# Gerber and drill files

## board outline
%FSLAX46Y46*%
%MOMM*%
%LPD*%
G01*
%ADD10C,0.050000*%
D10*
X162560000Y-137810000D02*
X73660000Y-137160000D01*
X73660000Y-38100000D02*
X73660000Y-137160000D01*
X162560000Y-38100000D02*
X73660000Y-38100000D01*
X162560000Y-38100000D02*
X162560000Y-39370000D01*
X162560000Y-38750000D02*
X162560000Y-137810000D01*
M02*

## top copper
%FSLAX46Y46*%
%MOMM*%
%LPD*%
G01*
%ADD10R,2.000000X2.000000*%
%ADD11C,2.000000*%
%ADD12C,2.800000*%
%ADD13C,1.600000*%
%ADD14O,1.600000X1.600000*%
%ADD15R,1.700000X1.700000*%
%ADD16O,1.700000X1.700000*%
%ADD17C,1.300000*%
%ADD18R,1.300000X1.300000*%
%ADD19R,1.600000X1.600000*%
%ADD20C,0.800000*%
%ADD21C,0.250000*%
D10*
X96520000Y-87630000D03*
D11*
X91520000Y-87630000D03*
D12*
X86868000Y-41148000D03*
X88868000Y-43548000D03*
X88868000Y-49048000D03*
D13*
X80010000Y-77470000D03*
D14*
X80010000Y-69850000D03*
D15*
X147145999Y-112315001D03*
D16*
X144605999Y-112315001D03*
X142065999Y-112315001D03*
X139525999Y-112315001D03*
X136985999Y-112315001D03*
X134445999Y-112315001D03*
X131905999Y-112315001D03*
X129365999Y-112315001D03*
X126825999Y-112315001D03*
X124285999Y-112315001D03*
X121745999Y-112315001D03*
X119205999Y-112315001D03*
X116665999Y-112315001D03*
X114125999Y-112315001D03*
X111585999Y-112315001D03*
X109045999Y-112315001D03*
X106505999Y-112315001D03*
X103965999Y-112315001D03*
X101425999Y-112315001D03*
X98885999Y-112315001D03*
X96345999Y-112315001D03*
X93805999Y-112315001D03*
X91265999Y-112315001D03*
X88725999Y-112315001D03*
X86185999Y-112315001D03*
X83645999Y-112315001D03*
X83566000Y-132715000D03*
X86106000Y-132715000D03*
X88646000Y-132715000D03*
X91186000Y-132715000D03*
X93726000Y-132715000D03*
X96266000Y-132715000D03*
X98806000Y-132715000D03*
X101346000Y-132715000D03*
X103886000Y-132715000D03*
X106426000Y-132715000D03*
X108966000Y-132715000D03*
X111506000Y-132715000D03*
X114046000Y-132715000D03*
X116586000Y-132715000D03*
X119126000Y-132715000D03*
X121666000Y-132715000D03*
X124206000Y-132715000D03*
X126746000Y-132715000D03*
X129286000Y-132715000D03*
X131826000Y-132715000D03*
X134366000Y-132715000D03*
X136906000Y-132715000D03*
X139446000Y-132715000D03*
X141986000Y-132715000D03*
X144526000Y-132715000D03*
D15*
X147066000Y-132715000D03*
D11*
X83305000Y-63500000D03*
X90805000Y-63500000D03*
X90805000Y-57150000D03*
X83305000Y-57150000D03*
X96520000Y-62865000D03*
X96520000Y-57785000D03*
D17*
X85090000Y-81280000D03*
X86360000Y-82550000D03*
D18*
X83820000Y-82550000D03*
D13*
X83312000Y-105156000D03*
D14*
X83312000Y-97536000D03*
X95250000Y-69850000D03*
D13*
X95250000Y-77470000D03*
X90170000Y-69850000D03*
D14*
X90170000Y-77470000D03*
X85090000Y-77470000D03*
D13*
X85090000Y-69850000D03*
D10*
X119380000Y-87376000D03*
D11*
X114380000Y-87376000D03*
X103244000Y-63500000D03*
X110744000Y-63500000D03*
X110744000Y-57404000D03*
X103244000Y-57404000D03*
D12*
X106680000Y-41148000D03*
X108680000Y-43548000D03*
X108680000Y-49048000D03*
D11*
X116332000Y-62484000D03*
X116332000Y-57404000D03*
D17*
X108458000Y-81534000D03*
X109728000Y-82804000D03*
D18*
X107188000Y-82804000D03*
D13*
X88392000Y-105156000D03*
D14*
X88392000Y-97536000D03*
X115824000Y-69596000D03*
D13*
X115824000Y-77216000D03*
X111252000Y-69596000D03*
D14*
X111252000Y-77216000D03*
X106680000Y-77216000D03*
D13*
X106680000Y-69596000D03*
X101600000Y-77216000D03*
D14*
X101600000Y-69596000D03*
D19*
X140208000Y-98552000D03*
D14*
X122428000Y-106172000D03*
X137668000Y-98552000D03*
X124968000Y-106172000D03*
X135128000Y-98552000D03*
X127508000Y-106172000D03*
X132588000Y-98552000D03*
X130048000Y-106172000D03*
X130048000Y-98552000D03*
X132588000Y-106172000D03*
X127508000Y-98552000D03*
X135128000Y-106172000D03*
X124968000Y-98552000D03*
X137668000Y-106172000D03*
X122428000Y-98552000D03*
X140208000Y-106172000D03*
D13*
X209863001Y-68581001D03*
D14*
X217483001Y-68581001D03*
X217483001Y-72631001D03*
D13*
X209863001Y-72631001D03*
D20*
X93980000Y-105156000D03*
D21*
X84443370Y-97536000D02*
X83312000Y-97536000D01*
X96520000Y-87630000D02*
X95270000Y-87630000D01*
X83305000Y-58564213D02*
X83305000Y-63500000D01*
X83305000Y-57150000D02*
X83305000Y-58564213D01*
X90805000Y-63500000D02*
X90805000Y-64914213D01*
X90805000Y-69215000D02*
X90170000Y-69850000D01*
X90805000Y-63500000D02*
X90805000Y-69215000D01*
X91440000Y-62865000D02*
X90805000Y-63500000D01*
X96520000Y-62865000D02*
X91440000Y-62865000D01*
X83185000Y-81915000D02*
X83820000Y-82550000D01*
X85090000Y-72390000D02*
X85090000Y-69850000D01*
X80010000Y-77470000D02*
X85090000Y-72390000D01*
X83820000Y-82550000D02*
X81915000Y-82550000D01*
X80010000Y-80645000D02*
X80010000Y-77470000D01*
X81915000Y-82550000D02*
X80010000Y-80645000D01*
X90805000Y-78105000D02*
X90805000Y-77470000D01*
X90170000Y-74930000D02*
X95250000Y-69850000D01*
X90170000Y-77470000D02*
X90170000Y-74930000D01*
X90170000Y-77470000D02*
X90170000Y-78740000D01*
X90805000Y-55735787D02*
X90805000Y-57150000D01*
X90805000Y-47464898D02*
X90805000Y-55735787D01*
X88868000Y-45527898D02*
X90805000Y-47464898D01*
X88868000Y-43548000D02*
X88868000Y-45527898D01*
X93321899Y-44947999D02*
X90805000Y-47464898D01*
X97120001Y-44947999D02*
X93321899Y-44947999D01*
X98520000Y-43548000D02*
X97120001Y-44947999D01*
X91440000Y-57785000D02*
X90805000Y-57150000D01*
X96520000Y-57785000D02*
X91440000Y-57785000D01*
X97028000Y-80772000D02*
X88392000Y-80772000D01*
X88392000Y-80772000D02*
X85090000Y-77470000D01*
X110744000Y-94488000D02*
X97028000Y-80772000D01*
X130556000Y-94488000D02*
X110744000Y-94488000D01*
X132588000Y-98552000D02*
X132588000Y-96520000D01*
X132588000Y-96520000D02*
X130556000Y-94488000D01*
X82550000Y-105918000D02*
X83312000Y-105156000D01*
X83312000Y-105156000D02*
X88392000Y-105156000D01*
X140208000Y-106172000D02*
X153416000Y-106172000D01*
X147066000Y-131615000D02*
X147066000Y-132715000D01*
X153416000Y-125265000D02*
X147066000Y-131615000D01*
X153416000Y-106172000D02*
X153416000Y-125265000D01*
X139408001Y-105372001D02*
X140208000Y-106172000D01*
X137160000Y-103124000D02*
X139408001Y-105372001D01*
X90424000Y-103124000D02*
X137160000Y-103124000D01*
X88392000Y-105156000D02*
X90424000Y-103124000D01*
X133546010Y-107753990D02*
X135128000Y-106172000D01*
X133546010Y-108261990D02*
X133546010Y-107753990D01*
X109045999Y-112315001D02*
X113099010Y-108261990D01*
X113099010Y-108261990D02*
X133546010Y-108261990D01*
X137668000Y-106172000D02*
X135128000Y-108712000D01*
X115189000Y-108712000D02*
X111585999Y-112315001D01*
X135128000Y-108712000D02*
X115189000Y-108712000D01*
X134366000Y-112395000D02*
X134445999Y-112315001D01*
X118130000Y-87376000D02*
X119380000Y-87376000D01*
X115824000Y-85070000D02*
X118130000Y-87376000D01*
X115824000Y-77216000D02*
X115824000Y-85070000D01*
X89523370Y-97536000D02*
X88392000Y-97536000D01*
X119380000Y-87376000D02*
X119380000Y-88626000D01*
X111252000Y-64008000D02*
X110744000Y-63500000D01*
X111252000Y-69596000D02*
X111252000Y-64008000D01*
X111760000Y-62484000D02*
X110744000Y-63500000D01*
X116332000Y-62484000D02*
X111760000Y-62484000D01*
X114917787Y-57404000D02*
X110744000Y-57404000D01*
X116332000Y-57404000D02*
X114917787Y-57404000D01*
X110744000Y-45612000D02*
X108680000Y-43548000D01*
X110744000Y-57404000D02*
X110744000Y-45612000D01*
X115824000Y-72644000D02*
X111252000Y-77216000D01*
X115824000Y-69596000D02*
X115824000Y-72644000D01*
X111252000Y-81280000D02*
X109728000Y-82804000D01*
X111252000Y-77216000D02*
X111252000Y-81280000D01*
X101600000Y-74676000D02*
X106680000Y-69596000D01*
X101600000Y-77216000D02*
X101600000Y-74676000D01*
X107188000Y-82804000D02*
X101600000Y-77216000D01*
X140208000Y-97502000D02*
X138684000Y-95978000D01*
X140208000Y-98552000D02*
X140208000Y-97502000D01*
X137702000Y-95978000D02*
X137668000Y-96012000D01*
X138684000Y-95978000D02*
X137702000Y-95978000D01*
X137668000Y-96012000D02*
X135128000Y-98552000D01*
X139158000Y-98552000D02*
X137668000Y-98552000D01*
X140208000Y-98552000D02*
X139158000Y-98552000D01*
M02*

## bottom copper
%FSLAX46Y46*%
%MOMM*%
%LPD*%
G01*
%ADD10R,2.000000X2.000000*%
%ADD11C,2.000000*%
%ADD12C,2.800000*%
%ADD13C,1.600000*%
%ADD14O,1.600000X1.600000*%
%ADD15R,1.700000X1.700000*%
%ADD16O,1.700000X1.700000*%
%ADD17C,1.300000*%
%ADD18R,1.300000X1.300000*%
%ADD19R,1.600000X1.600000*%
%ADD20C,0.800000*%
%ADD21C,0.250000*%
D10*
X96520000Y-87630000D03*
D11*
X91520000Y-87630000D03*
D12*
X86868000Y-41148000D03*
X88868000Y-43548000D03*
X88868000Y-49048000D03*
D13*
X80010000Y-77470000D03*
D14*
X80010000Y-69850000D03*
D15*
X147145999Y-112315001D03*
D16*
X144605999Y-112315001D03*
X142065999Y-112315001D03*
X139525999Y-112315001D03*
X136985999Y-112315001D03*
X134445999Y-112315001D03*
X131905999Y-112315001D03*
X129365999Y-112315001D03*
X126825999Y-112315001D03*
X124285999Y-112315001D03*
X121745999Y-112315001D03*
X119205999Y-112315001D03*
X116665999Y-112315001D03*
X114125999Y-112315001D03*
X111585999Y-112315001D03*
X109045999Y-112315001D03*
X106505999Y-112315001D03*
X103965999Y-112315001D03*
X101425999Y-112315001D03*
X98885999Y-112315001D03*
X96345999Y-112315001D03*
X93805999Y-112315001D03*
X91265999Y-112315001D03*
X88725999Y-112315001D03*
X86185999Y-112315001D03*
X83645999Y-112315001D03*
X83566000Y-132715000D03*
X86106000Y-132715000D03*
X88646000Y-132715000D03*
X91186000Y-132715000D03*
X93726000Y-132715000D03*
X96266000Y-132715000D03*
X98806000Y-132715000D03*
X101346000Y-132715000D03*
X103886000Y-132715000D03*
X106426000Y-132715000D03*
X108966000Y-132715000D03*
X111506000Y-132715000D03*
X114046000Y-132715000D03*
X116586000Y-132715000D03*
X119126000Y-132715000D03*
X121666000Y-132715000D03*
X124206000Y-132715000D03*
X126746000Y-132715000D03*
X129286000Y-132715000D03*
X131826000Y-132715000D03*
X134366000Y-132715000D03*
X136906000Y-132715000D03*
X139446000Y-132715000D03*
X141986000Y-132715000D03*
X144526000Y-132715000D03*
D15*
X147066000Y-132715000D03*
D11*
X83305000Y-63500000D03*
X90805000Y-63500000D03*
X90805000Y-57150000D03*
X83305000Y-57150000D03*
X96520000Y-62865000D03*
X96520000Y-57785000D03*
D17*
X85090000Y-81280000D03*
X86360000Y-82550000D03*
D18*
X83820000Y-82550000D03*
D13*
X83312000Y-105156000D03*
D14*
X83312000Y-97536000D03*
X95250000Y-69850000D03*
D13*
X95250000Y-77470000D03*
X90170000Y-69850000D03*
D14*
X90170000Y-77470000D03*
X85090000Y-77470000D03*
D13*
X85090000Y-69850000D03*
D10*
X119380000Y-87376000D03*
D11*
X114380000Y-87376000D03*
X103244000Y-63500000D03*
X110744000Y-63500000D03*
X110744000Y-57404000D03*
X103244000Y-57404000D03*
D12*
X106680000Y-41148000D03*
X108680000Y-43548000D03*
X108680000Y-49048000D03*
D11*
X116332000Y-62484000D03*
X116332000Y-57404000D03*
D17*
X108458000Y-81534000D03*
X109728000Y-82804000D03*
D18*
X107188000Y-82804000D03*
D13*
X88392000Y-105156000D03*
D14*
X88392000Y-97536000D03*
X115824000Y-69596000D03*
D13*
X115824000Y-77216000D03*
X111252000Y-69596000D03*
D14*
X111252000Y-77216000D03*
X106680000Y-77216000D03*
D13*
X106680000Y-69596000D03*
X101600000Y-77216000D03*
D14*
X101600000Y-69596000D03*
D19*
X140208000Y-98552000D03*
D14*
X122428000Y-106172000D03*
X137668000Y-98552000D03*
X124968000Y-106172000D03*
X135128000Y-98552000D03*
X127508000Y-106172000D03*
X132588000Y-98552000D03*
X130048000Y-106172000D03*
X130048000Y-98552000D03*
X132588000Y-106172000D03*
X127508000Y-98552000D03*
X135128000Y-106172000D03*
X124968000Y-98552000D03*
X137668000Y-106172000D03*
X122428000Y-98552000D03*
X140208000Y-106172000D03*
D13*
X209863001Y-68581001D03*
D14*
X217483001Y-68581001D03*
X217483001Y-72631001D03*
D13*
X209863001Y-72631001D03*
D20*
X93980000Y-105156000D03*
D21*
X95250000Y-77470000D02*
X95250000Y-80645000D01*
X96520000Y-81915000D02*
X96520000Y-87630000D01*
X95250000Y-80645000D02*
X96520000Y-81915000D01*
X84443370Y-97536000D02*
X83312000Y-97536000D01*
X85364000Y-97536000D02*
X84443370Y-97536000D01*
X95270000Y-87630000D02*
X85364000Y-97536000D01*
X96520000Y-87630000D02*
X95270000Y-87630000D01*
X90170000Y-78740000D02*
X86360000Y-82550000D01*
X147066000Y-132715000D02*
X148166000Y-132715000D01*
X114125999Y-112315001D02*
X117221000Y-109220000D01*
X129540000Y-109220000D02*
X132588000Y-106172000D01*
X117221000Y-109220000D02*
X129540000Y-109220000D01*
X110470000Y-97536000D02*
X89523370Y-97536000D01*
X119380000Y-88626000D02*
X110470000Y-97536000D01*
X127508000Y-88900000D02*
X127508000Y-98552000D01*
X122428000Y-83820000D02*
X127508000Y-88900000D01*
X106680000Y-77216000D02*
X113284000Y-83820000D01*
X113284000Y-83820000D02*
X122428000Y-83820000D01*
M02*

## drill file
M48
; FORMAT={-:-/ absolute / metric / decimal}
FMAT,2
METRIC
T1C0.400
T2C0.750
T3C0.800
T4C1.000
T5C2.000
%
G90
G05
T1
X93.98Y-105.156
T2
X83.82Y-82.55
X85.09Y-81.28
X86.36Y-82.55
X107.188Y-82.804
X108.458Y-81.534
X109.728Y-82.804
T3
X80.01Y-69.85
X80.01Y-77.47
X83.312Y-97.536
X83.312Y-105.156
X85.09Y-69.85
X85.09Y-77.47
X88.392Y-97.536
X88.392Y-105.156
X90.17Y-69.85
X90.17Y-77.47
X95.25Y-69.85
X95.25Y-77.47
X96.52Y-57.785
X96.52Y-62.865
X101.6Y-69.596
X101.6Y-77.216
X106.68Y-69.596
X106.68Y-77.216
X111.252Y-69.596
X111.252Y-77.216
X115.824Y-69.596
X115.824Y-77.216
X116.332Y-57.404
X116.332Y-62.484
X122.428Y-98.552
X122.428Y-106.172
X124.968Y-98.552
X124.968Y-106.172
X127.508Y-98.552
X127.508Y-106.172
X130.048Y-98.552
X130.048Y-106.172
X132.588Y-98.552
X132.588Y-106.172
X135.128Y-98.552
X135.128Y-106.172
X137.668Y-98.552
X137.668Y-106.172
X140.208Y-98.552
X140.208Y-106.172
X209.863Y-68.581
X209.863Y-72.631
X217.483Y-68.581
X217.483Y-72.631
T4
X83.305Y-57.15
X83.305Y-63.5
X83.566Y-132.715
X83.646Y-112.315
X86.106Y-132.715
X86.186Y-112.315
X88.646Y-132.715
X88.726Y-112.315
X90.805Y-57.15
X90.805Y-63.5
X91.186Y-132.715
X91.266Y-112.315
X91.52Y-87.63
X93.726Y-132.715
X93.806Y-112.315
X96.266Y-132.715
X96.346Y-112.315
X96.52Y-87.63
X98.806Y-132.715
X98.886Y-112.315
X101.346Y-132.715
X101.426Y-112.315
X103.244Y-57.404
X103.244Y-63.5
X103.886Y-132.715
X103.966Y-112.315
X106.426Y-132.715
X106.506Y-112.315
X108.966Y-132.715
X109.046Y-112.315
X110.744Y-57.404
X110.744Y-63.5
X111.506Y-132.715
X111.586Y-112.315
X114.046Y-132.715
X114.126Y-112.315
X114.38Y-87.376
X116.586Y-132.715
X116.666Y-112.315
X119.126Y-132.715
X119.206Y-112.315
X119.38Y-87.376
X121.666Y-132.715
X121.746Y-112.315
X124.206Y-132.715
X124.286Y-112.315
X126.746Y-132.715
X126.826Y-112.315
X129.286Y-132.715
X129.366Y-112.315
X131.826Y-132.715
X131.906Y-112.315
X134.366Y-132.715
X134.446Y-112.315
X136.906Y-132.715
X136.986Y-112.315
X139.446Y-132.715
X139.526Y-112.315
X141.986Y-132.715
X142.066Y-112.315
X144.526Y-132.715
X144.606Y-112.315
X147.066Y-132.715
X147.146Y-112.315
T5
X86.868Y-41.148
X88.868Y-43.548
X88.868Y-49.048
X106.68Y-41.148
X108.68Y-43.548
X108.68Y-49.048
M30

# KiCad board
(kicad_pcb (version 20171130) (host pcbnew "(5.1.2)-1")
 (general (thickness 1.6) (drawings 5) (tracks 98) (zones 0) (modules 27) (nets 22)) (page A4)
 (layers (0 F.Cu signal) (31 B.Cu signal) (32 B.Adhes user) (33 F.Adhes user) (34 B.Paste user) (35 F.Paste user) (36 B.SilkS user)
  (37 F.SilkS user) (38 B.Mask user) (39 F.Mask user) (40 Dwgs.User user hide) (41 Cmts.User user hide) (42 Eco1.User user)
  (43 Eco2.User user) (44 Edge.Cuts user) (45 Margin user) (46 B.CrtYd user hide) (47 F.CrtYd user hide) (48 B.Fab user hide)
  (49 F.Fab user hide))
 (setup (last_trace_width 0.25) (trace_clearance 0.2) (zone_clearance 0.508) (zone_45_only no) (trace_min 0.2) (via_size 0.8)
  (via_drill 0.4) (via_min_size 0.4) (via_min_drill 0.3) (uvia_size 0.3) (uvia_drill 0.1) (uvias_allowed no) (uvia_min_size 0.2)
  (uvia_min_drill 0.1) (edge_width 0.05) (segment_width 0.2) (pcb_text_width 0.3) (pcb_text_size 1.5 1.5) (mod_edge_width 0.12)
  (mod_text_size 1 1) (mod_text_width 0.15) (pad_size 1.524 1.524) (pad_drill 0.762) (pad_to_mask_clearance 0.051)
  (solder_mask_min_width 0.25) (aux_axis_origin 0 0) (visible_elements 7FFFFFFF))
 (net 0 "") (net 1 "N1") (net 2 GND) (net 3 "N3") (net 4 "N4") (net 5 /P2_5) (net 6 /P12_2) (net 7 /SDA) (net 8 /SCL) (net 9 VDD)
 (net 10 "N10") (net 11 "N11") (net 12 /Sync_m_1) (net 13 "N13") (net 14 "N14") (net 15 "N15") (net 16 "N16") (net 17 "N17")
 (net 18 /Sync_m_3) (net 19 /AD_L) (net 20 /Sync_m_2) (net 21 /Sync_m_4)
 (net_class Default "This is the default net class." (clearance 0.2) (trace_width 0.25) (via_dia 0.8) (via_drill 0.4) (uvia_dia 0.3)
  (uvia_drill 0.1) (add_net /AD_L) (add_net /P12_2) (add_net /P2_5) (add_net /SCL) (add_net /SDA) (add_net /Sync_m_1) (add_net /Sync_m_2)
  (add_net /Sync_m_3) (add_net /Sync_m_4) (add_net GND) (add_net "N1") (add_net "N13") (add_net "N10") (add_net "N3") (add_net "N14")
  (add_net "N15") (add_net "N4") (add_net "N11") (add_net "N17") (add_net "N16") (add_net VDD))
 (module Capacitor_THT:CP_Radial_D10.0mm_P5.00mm (layer F.Cu) (at 96.52 87.63 180)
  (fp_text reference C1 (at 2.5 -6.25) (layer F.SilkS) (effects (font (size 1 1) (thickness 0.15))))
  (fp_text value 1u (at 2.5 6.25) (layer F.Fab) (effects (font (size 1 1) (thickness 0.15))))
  (pad 1 thru_hole rect (at 0 0 180) (size 2 2) (drill 1) (layers *.Cu *.Mask) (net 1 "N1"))
  (pad 2 thru_hole circle (at 5 0 180) (size 2 2) (drill 1) (layers *.Cu *.Mask) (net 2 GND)))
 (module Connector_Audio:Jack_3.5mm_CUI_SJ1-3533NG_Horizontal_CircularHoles (layer F.Cu) (at 86.868 41.148)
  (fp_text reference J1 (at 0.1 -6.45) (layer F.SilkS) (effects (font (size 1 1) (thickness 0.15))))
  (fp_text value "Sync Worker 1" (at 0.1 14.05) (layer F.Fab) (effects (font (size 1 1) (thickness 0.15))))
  (pad S thru_hole circle (at 0 0) (size 2.8 2.8) (drill 2) (layers *.Cu *.Mask) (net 2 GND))
  (pad T thru_hole circle (at 2 2.4) (size 2.8 2.8) (drill 2) (layers *.Cu *.Mask) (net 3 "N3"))
  (pad R thru_hole circle (at 2 7.9) (size 2.8 2.8) (drill 2) (layers *.Cu *.Mask)))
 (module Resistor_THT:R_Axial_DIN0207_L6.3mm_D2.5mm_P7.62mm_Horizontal (layer F.Cu) (at 80.01 77.47 90)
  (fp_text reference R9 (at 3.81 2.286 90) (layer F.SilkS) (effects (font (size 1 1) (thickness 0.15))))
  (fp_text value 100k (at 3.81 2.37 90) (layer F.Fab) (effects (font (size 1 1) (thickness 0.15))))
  (pad 1 thru_hole circle (at 0 0 90) (size 1.6 1.6) (drill 0.8) (layers *.Cu *.Mask) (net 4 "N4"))
  (pad 2 thru_hole oval (at 7.62 0 90) (size 1.6 1.6) (drill 0.8) (layers *.Cu *.Mask) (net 2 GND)))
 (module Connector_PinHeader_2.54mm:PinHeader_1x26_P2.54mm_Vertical (layer F.Cu) (at 147.145999 112.315001 270)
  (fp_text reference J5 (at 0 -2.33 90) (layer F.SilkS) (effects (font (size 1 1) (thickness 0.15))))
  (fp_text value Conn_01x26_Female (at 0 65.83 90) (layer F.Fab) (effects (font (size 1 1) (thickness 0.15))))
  (pad 1 thru_hole rect (at 0 0 270) (size 1.7 1.7) (drill 1) (layers *.Cu *.Mask))
  (pad 2 thru_hole oval (at 0 2.54 270) (size 1.7 1.7) (drill 1) (layers *.Cu *.Mask))
  (pad 3 thru_hole oval (at 0 5.08 270) (size 1.7 1.7) (drill 1) (layers *.Cu *.Mask))
  (pad 4 thru_hole oval (at 0 7.62 270) (size 1.7 1.7) (drill 1) (layers *.Cu *.Mask))
  (pad 5 thru_hole oval (at 0 10.16 270) (size 1.7 1.7) (drill 1) (layers *.Cu *.Mask))
  (pad 6 thru_hole oval (at 0 12.7 270) (size 1.7 1.7) (drill 1) (layers *.Cu *.Mask) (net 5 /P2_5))
  (pad 7 thru_hole oval (at 0 15.24 270) (size 1.7 1.7) (drill 1) (layers *.Cu *.Mask))
  (pad 8 thru_hole oval (at 0 17.78 270) (size 1.7 1.7) (drill 1) (layers *.Cu *.Mask))
  (pad 9 thru_hole oval (at 0 20.32 270) (size 1.7 1.7) (drill 1) (layers *.Cu *.Mask))
  (pad 10 thru_hole oval (at 0 22.86 270) (size 1.7 1.7) (drill 1) (layers *.Cu *.Mask))
  (pad 11 thru_hole oval (at 0 25.4 270) (size 1.7 1.7) (drill 1) (layers *.Cu *.Mask))
  (pad 12 thru_hole oval (at 0 27.94 270) (size 1.7 1.7) (drill 1) (layers *.Cu *.Mask))
  (pad 13 thru_hole oval (at 0 30.48 270) (size 1.7 1.7) (drill 1) (layers *.Cu *.Mask))
  (pad 14 thru_hole oval (at 0 33.02 270) (size 1.7 1.7) (drill 1) (layers *.Cu *.Mask) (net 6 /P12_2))
  (pad 15 thru_hole oval (at 0 35.56 270) (size 1.7 1.7) (drill 1) (layers *.Cu *.Mask) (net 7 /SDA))
  (pad 16 thru_hole oval (at 0 38.1 270) (size 1.7 1.7) (drill 1) (layers *.Cu *.Mask) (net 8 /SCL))
  (pad 17 thru_hole oval (at 0 40.64 270) (size 1.7 1.7) (drill 1) (layers *.Cu *.Mask))
  (pad 18 thru_hole oval (at 0 43.18 270) (size 1.7 1.7) (drill 1) (layers *.Cu *.Mask))
  (pad 19 thru_hole oval (at 0 45.72 270) (size 1.7 1.7) (drill 1) (layers *.Cu *.Mask))
  (pad 20 thru_hole oval (at 0 48.26 270) (size 1.7 1.7) (drill 1) (layers *.Cu *.Mask))
  (pad 21 thru_hole oval (at 0 50.8 270) (size 1.7 1.7) (drill 1) (layers *.Cu *.Mask))
  (pad 22 thru_hole oval (at 0 53.34 270) (size 1.7 1.7) (drill 1) (layers *.Cu *.Mask))
  (pad 23 thru_hole oval (at 0 55.88 270) (size 1.7 1.7) (drill 1) (layers *.Cu *.Mask))
  (pad 24 thru_hole oval (at 0 58.42 270) (size 1.7 1.7) (drill 1) (layers *.Cu *.Mask))
  (pad 25 thru_hole oval (at 0 60.96 270) (size 1.7 1.7) (drill 1) (layers *.Cu *.Mask) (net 2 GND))
  (pad 26 thru_hole oval (at 0 63.5 270) (size 1.7 1.7) (drill 1) (layers *.Cu *.Mask)))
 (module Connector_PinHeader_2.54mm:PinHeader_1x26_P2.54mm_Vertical (layer F.Cu) (at 147.066 132.715 270)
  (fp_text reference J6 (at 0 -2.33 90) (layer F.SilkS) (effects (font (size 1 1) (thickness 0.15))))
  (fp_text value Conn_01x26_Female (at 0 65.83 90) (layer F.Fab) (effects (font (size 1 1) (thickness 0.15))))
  (pad 26 thru_hole oval (at 0 63.5 270) (size 1.7 1.7) (drill 1) (layers *.Cu *.Mask) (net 2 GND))
  (pad 25 thru_hole oval (at 0 60.96 270) (size 1.7 1.7) (drill 1) (layers *.Cu *.Mask))
  (pad 24 thru_hole oval (at 0 58.42 270) (size 1.7 1.7) (drill 1) (layers *.Cu *.Mask))
  (pad 23 thru_hole oval (at 0 55.88 270) (size 1.7 1.7) (drill 1) (layers *.Cu *.Mask))
  (pad 22 thru_hole oval (at 0 53.34 270) (size 1.7 1.7) (drill 1) (layers *.Cu *.Mask))
  (pad 21 thru_hole oval (at 0 50.8 270) (size 1.7 1.7) (drill 1) (layers *.Cu *.Mask))
  (pad 20 thru_hole oval (at 0 48.26 270) (size 1.7 1.7) (drill 1) (layers *.Cu *.Mask))
  (pad 19 thru_hole oval (at 0 45.72 270) (size 1.7 1.7) (drill 1) (layers *.Cu *.Mask))
  (pad 18 thru_hole oval (at 0 43.18 270) (size 1.7 1.7) (drill 1) (layers *.Cu *.Mask))
  (pad 17 thru_hole oval (at 0 40.64 270) (size 1.7 1.7) (drill 1) (layers *.Cu *.Mask))
  (pad 16 thru_hole oval (at 0 38.1 270) (size 1.7 1.7) (drill 1) (layers *.Cu *.Mask))
  (pad 15 thru_hole oval (at 0 35.56 270) (size 1.7 1.7) (drill 1) (layers *.Cu *.Mask))
  (pad 14 thru_hole oval (at 0 33.02 270) (size 1.7 1.7) (drill 1) (layers *.Cu *.Mask))
  (pad 13 thru_hole oval (at 0 30.48 270) (size 1.7 1.7) (drill 1) (layers *.Cu *.Mask))
  (pad 12 thru_hole oval (at 0 27.94 270) (size 1.7 1.7) (drill 1) (layers *.Cu *.Mask))
  (pad 11 thru_hole oval (at 0 25.4 270) (size 1.7 1.7) (drill 1) (layers *.Cu *.Mask))
  (pad 10 thru_hole oval (at 0 22.86 270) (size 1.7 1.7) (drill 1) (layers *.Cu *.Mask))
  (pad 9 thru_hole oval (at 0 20.32 270) (size 1.7 1.7) (drill 1) (layers *.Cu *.Mask))
  (pad 8 thru_hole oval (at 0 17.78 270) (size 1.7 1.7) (drill 1) (layers *.Cu *.Mask))
  (pad 7 thru_hole oval (at 0 15.24 270) (size 1.7 1.7) (drill 1) (layers *.Cu *.Mask))
  (pad 6 thru_hole oval (at 0 12.7 270) (size 1.7 1.7) (drill 1) (layers *.Cu *.Mask) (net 5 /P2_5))
  (pad 5 thru_hole oval (at 0 10.16 270) (size 1.7 1.7) (drill 1) (layers *.Cu *.Mask))
  (pad 4 thru_hole oval (at 0 7.62 270) (size 1.7 1.7) (drill 1) (layers *.Cu *.Mask))
  (pad 3 thru_hole oval (at 0 5.08 270) (size 1.7 1.7) (drill 1) (layers *.Cu *.Mask))
  (pad 2 thru_hole oval (at 0 2.54 270) (size 1.7 1.7) (drill 1) (layers *.Cu *.Mask) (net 2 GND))
  (pad 1 thru_hole rect (at 0 0 270) (size 1.7 1.7) (drill 1) (layers *.Cu *.Mask) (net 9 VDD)))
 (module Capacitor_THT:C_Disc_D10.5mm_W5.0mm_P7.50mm (layer F.Cu) (at 90.805 63.5 180)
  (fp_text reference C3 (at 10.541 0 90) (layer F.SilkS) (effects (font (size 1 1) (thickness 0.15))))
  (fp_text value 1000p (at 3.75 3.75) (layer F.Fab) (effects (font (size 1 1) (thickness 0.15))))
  (pad 2 thru_hole circle (at 7.5 0 180) (size 2 2) (drill 1) (layers *.Cu *.Mask) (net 2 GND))
  (pad 1 thru_hole circle (at 0 0 180) (size 2 2) (drill 1) (layers *.Cu *.Mask) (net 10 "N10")))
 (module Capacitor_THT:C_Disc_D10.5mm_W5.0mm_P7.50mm (layer F.Cu) (at 90.805 57.15 180)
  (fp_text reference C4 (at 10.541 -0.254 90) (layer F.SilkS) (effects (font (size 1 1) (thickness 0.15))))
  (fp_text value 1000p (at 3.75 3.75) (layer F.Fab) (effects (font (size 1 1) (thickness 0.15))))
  (pad 1 thru_hole circle (at 0 0 180) (size 2 2) (drill 1) (layers *.Cu *.Mask) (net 3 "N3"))
  (pad 2 thru_hole circle (at 7.5 0 180) (size 2 2) (drill 1) (layers *.Cu *.Mask) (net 2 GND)))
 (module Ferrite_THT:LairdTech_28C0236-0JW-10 (layer F.Cu) (at 96.52 57.785 270)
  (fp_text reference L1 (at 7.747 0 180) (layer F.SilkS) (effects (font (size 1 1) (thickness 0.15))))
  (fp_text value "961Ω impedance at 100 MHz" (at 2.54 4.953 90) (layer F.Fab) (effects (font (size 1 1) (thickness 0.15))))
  (pad 2 thru_hole circle (at 5.08 0 270) (size 2 2) (drill 0.8) (layers *.Cu *.Mask) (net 10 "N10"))
  (pad 1 thru_hole circle (at 0 0 270) (size 2 2) (drill 0.8) (layers *.Cu *.Mask) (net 3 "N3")))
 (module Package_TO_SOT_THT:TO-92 (layer F.Cu) (at 83.82 82.55)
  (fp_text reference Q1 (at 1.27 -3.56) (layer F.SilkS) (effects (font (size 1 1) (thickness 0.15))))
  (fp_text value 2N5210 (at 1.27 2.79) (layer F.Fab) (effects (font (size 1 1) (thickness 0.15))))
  (pad 2 thru_hole circle (at 1.27 -1.27 90) (size 1.3 1.3) (drill 0.75) (layers *.Cu *.Mask) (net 2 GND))
  (pad 3 thru_hole circle (at 2.54 0 90) (size 1.3 1.3) (drill 0.75) (layers *.Cu *.Mask) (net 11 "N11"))
  (pad 1 thru_hole rect (at 0 0 90) (size 1.3 1.3) (drill 0.75) (layers *.Cu *.Mask) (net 4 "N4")))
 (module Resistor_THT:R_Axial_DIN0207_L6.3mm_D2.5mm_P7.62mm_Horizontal (layer F.Cu) (at 83.312 105.156 90)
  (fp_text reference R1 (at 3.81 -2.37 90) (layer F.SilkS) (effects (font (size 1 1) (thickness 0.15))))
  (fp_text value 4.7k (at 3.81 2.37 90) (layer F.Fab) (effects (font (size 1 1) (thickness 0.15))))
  (pad 1 thru_hole circle (at 0 0 90) (size 1.6 1.6) (drill 0.8) (layers *.Cu *.Mask) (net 9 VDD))
  (pad 2 thru_hole oval (at 7.62 0 90) (size 1.6 1.6) (drill 0.8) (layers *.Cu *.Mask) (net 1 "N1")))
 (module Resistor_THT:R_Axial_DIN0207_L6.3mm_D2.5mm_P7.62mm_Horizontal (layer F.Cu) (at 95.25 77.47 90)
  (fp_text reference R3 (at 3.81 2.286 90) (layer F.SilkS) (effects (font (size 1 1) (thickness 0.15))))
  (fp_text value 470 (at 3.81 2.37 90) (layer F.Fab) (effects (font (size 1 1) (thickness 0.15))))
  (pad 2 thru_hole oval (at 7.62 0 90) (size 1.6 1.6) (drill 0.8) (layers *.Cu *.Mask) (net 11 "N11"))
  (pad 1 thru_hole circle (at 0 0 90) (size 1.6 1.6) (drill 0.8) (layers *.Cu *.Mask) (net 1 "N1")))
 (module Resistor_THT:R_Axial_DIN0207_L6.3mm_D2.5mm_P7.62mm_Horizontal (layer F.Cu) (at 90.17 69.85 270)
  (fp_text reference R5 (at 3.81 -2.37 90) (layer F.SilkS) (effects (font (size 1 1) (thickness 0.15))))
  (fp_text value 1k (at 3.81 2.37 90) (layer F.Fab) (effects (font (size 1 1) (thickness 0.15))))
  (pad 1 thru_hole circle (at 0 0 270) (size 1.6 1.6) (drill 0.8) (layers *.Cu *.Mask) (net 10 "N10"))
  (pad 2 thru_hole oval (at 7.62 0 270) (size 1.6 1.6) (drill 0.8) (layers *.Cu *.Mask) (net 11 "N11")))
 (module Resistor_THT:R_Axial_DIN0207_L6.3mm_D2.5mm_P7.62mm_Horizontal (layer F.Cu) (at 85.09 69.85 270)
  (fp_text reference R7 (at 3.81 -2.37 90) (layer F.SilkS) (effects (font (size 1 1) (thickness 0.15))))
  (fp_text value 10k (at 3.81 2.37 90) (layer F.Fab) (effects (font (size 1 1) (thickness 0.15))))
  (pad 2 thru_hole oval (at 7.62 0 270) (size 1.6 1.6) (drill 0.8) (layers *.Cu *.Mask) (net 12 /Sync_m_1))
  (pad 1 thru_hole circle (at 0 0 270) (size 1.6 1.6) (drill 0.8) (layers *.Cu *.Mask) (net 4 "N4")))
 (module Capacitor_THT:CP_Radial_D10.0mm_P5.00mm (layer F.Cu) (at 119.38 87.376 180)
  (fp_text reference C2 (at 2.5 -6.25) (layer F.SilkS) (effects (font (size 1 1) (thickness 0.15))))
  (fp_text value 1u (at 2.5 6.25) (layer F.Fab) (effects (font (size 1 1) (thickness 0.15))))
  (pad 1 thru_hole rect (at 0 0 180) (size 2 2) (drill 1) (layers *.Cu *.Mask) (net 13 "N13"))
  (pad 2 thru_hole circle (at 5 0 180) (size 2 2) (drill 1) (layers *.Cu *.Mask) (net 2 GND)))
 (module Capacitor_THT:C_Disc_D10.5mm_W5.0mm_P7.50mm (layer F.Cu) (at 110.744 63.5 180)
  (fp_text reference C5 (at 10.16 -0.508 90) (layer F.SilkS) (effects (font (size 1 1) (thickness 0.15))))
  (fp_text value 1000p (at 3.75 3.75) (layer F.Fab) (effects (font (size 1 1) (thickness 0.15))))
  (pad 2 thru_hole circle (at 7.5 0 180) (size 2 2) (drill 1) (layers *.Cu *.Mask) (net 2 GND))
  (pad 1 thru_hole circle (at 0 0 180) (size 2 2) (drill 1) (layers *.Cu *.Mask) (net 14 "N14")))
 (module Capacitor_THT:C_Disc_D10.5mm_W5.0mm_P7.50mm (layer F.Cu) (at 110.744 57.404 180)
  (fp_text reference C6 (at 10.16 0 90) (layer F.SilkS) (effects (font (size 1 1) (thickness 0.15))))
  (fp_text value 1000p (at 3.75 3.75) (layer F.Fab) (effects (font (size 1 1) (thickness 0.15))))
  (pad 1 thru_hole circle (at 0 0 180) (size 2 2) (drill 1) (layers *.Cu *.Mask) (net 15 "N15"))
  (pad 2 thru_hole circle (at 7.5 0 180) (size 2 2) (drill 1) (layers *.Cu *.Mask) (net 2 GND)))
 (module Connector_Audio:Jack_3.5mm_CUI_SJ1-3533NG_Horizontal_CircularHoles (layer F.Cu) (at 106.68 41.148)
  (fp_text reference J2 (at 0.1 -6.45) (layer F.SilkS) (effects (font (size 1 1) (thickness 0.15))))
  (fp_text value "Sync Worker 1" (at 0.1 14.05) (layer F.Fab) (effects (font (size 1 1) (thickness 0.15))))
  (pad S thru_hole circle (at 0 0) (size 2.8 2.8) (drill 2) (layers *.Cu *.Mask) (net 2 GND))
  (pad T thru_hole circle (at 2 2.4) (size 2.8 2.8) (drill 2) (layers *.Cu *.Mask) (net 15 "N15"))
  (pad R thru_hole circle (at 2 7.9) (size 2.8 2.8) (drill 2) (layers *.Cu *.Mask)))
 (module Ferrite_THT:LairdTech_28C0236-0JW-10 (layer F.Cu) (at 116.332 57.404 270)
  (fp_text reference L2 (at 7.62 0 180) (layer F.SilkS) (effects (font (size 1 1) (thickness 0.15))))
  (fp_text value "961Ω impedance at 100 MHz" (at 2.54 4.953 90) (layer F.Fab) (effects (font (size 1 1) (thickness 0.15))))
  (pad 2 thru_hole circle (at 5.08 0 270) (size 2 2) (drill 0.8) (layers *.Cu *.Mask) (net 14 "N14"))
  (pad 1 thru_hole circle (at 0 0 270) (size 2 2) (drill 0.8) (layers *.Cu *.Mask) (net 15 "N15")))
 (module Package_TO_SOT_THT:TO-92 (layer F.Cu) (at 107.188 82.804)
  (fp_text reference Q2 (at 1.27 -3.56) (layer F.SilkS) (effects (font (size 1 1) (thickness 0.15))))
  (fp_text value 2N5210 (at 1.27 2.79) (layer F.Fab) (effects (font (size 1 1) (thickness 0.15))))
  (pad 2 thru_hole circle (at 1.27 -1.27 90) (size 1.3 1.3) (drill 0.75) (layers *.Cu *.Mask) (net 2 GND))
  (pad 3 thru_hole circle (at 2.54 0 90) (size 1.3 1.3) (drill 0.75) (layers *.Cu *.Mask) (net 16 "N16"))
  (pad 1 thru_hole rect (at 0 0 90) (size 1.3 1.3) (drill 0.75) (layers *.Cu *.Mask) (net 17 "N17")))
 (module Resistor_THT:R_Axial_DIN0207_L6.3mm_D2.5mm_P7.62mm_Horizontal (layer F.Cu) (at 88.392 105.156 90)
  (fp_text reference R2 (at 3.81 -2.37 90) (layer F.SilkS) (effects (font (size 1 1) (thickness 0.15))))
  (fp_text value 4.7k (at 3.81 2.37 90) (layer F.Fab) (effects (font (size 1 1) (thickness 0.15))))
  (pad 1 thru_hole circle (at 0 0 90) (size 1.6 1.6) (drill 0.8) (layers *.Cu *.Mask) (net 9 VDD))
  (pad 2 thru_hole oval (at 7.62 0 90) (size 1.6 1.6) (drill 0.8) (layers *.Cu *.Mask) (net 13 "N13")))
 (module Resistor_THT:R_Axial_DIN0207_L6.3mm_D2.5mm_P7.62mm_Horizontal (layer F.Cu) (at 115.824 77.216 90)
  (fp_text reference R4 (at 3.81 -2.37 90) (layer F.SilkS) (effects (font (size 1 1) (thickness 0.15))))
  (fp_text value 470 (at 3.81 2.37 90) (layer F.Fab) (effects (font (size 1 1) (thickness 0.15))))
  (pad 2 thru_hole oval (at 7.62 0 90) (size 1.6 1.6) (drill 0.8) (layers *.Cu *.Mask) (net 16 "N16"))
  (pad 1 thru_hole circle (at 0 0 90) (size 1.6 1.6) (drill 0.8) (layers *.Cu *.Mask) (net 13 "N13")))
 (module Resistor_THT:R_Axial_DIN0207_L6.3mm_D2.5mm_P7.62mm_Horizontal (layer F.Cu) (at 111.252 69.596 270)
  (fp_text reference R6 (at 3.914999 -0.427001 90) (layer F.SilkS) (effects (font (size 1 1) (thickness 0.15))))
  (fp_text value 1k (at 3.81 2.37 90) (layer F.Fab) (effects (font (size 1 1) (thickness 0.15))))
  (pad 1 thru_hole circle (at 0 0 270) (size 1.6 1.6) (drill 0.8) (layers *.Cu *.Mask) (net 14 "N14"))
  (pad 2 thru_hole oval (at 7.62 0 270) (size 1.6 1.6) (drill 0.8) (layers *.Cu *.Mask) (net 16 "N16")))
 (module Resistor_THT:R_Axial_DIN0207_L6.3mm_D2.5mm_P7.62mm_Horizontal (layer F.Cu) (at 106.68 69.596 270)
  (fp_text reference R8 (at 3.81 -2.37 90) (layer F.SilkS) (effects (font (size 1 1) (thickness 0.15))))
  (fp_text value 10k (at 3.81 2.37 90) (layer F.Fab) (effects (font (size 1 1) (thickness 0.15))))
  (pad 2 thru_hole oval (at 7.62 0 270) (size 1.6 1.6) (drill 0.8) (layers *.Cu *.Mask) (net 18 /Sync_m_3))
  (pad 1 thru_hole circle (at 0 0 270) (size 1.6 1.6) (drill 0.8) (layers *.Cu *.Mask) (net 17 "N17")))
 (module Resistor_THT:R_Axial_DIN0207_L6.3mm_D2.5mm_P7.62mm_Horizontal (layer F.Cu) (at 101.6 77.216 90)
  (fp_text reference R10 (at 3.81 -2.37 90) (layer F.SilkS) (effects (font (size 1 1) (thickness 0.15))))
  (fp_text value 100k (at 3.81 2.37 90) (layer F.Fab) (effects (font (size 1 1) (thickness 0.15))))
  (pad 1 thru_hole circle (at 0 0 90) (size 1.6 1.6) (drill 0.8) (layers *.Cu *.Mask) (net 17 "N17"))
  (pad 2 thru_hole oval (at 7.62 0 90) (size 1.6 1.6) (drill 0.8) (layers *.Cu *.Mask) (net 2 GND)))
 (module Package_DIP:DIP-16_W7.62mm (layer F.Cu) (at 140.208 98.552 270)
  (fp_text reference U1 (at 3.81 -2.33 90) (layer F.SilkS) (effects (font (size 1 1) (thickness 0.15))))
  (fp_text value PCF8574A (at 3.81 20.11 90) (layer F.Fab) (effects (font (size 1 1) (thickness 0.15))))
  (pad 1 thru_hole rect (at 0 0 270) (size 1.6 1.6) (drill 0.8) (layers *.Cu *.Mask) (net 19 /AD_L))
  (pad 9 thru_hole oval (at 7.62 17.78 270) (size 1.6 1.6) (drill 0.8) (layers *.Cu *.Mask))
  (pad 2 thru_hole oval (at 0 2.54 270) (size 1.6 1.6) (drill 0.8) (layers *.Cu *.Mask) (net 19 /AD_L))
  (pad 10 thru_hole oval (at 7.62 15.24 270) (size 1.6 1.6) (drill 0.8) (layers *.Cu *.Mask))
  (pad 3 thru_hole oval (at 0 5.08 270) (size 1.6 1.6) (drill 0.8) (layers *.Cu *.Mask) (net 19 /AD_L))
  (pad 11 thru_hole oval (at 7.62 12.7 270) (size 1.6 1.6) (drill 0.8) (layers *.Cu *.Mask))
  (pad 4 thru_hole oval (at 0 7.62 270) (size 1.6 1.6) (drill 0.8) (layers *.Cu *.Mask) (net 12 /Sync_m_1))
  (pad 12 thru_hole oval (at 7.62 10.16 270) (size 1.6 1.6) (drill 0.8) (layers *.Cu *.Mask))
  (pad 5 thru_hole oval (at 0 10.16 270) (size 1.6 1.6) (drill 0.8) (layers *.Cu *.Mask) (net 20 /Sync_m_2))
  (pad 13 thru_hole oval (at 7.62 7.62 270) (size 1.6 1.6) (drill 0.8) (layers *.Cu *.Mask) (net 6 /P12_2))
  (pad 6 thru_hole oval (at 0 12.7 270) (size 1.6 1.6) (drill 0.8) (layers *.Cu *.Mask) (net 18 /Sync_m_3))
  (pad 14 thru_hole oval (at 7.62 5.08 270) (size 1.6 1.6) (drill 0.8) (layers *.Cu *.Mask) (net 8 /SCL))
  (pad 7 thru_hole oval (at 0 15.24 270) (size 1.6 1.6) (drill 0.8) (layers *.Cu *.Mask) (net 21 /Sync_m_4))
  (pad 15 thru_hole oval (at 7.62 2.54 270) (size 1.6 1.6) (drill 0.8) (layers *.Cu *.Mask) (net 7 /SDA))
  (pad 8 thru_hole oval (at 0 17.78 270) (size 1.6 1.6) (drill 0.8) (layers *.Cu *.Mask) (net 2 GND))
  (pad 16 thru_hole oval (at 7.62 0 270) (size 1.6 1.6) (drill 0.8) (layers *.Cu *.Mask) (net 9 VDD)))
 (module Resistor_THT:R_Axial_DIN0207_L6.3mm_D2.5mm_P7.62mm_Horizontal (layer F.Cu) (at 209.863001 68.581001)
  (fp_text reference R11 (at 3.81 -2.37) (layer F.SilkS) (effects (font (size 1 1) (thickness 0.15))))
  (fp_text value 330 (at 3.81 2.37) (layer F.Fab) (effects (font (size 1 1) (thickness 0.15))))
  (pad 1 thru_hole circle (at 0 0) (size 1.6 1.6) (drill 0.8) (layers *.Cu *.Mask) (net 20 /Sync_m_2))
  (pad 2 thru_hole oval (at 7.62 0) (size 1.6 1.6) (drill 0.8) (layers *.Cu *.Mask)))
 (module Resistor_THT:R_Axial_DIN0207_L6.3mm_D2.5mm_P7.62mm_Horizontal (layer F.Cu) (at 209.863001 72.631001)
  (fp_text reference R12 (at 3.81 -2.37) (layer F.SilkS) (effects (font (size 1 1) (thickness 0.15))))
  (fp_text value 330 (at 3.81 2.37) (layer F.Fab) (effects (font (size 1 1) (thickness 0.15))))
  (pad 2 thru_hole oval (at 7.62 0) (size 1.6 1.6) (drill 0.8) (layers *.Cu *.Mask))
  (pad 1 thru_hole circle (at 0 0) (size 1.6 1.6) (drill 0.8) (layers *.Cu *.Mask) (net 21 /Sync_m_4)))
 (gr_line (start 162.56 137.81) (end 73.66 137.16) (layer Edge.Cuts) (width 0.05))
 (gr_line (start 73.66 38.1) (end 73.66 137.16) (layer Edge.Cuts) (width 0.05))
 (gr_line (start 162.56 38.1) (end 73.66 38.1) (layer Edge.Cuts) (width 0.05))
 (gr_line (start 162.56 38.1) (end 162.56 39.37) (layer Edge.Cuts) (width 0.05))
 (gr_line (start 162.56 38.75) (end 162.56 137.81) (layer Edge.Cuts) (width 0.05))
 (via (at 93.98 105.156) (size 0.8) (drill 0.4) (layers F.Cu B.Cu) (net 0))
 (segment (start 95.25 77.47) (end 95.25 80.645) (width 0.25) (layer B.Cu) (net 1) (status 10))
 (segment (start 96.52 81.915) (end 96.52 87.63) (width 0.25) (layer B.Cu) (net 1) (status 20))
 (segment (start 95.25 80.645) (end 96.52 81.915) (width 0.25) (layer B.Cu) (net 1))
 (segment (start 84.44337 97.536) (end 83.312 97.536) (width 0.25) (layer F.Cu) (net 1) (status 20))
 (segment (start 96.52 87.63) (end 95.27 87.63) (width 0.25) (layer F.Cu) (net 1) (status 10))
 (segment (start 84.44337 97.536) (end 83.312 97.536) (width 0.25) (layer B.Cu) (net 1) (status 20))
 (segment (start 85.364 97.536) (end 84.44337 97.536) (width 0.25) (layer B.Cu) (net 1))
 (segment (start 95.27 87.63) (end 85.364 97.536) (width 0.25) (layer B.Cu) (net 1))
 (segment (start 96.52 87.63) (end 95.27 87.63) (width 0.25) (layer B.Cu) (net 1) (status 10))
 (segment (start 83.305 58.564213) (end 83.305 63.5) (width 0.25) (layer F.Cu) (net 2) (status 20))
 (segment (start 83.305 57.15) (end 83.305 58.564213) (width 0.25) (layer F.Cu) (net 2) (status 10))
 (segment (start 90.805 63.5) (end 90.805 64.914213) (width 0.25) (layer F.Cu) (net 10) (status 10))
 (segment (start 90.805 69.215) (end 90.17 69.85) (width 0.25) (layer F.Cu) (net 10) (status 20))
 (segment (start 90.805 63.5) (end 90.805 69.215) (width 0.25) (layer F.Cu) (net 10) (status 10))
 (segment (start 91.44 62.865) (end 90.805 63.5) (width 0.25) (layer F.Cu) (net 10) (status 30))
 (segment (start 96.52 62.865) (end 91.44 62.865) (width 0.25) (layer F.Cu) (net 10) (status 30))
 (segment (start 83.185 81.915) (end 83.82 82.55) (width 0.25) (layer F.Cu) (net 4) (status 30))
 (segment (start 85.09 72.39) (end 85.09 69.85) (width 0.25) (layer F.Cu) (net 4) (status 20))
 (segment (start 80.01 77.47) (end 85.09 72.39) (width 0.25) (layer F.Cu) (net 4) (status 10))
 (segment (start 83.82 82.55) (end 81.915 82.55) (width 0.25) (layer F.Cu) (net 4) (status 10))
 (segment (start 80.01 80.645) (end 80.01 77.47) (width 0.25) (layer F.Cu) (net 4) (status 20))
 (segment (start 81.915 82.55) (end 80.01 80.645) (width 0.25) (layer F.Cu) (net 4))
 (segment (start 90.805 78.105) (end 90.805 77.47) (width 0.25) (layer F.Cu) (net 11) (status 30))
 (segment (start 90.17 74.93) (end 95.25 69.85) (width 0.25) (layer F.Cu) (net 11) (status 20))
 (segment (start 90.17 77.47) (end 90.17 74.93) (width 0.25) (layer F.Cu) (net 11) (status 10))
 (segment (start 90.17 78.74) (end 86.36 82.55) (width 0.25) (layer B.Cu) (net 11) (status 20))
 (segment (start 90.17 77.47) (end 90.17 78.74) (width 0.25) (layer F.Cu) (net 11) (status 10))
 (segment (start 90.805 55.735787) (end 90.805 57.15) (width 0.25) (layer F.Cu) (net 3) (status 20))
 (segment (start 90.805 47.464898) (end 90.805 55.735787) (width 0.25) (layer F.Cu) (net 3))
 (segment (start 88.868 45.527898) (end 90.805 47.464898) (width 0.25) (layer F.Cu) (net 3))
 (segment (start 88.868 43.548) (end 88.868 45.527898) (width 0.25) (layer F.Cu) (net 3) (status 10))
 (segment (start 93.321899 44.947999) (end 90.805 47.464898) (width 0.25) (layer F.Cu) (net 3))
 (segment (start 97.120001 44.947999) (end 93.321899 44.947999) (width 0.25) (layer F.Cu) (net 3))
 (segment (start 98.52 43.548) (end 97.120001 44.947999) (width 0.25) (layer F.Cu) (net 3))
 (segment (start 91.44 57.785) (end 90.805 57.15) (width 0.25) (layer F.Cu) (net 3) (status 30))
 (segment (start 96.52 57.785) (end 91.44 57.785) (width 0.25) (layer F.Cu) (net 3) (status 30))
 (segment (start 97.028 80.772) (end 88.392 80.772) (width 0.25) (layer F.Cu) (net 12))
 (segment (start 88.392 80.772) (end 85.09 77.47) (width 0.25) (layer F.Cu) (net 12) (status 20))
 (segment (start 110.744 94.488) (end 97.028 80.772) (width 0.25) (layer F.Cu) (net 12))
 (segment (start 130.556 94.488) (end 110.744 94.488) (width 0.25) (layer F.Cu) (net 12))
 (segment (start 132.588 98.552) (end 132.588 96.52) (width 0.25) (layer F.Cu) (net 12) (status 10))
 (segment (start 132.588 96.52) (end 130.556 94.488) (width 0.25) (layer F.Cu) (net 12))
 (segment (start 82.55 105.918) (end 83.312 105.156) (width 0.25) (layer F.Cu) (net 9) (status 20))
 (segment (start 83.312 105.156) (end 88.392 105.156) (width 0.25) (layer F.Cu) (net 9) (status 30))
 (segment (start 147.066 132.715) (end 148.166 132.715) (width 0.25) (layer B.Cu) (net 9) (status 10))
 (segment (start 140.208 106.172) (end 153.416 106.172) (width 0.25) (layer F.Cu) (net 9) (status 10))
 (segment (start 147.066 131.615) (end 147.066 132.715) (width 0.25) (layer F.Cu) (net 9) (status 20))
 (segment (start 153.416 125.265) (end 147.066 131.615) (width 0.25) (layer F.Cu) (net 9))
 (segment (start 153.416 106.172) (end 153.416 125.265) (width 0.25) (layer F.Cu) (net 9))
 (segment (start 139.408001 105.372001) (end 140.208 106.172) (width 0.25) (layer F.Cu) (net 9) (status 30))
 (segment (start 137.16 103.124) (end 139.408001 105.372001) (width 0.25) (layer F.Cu) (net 9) (status 20))
 (segment (start 90.424 103.124) (end 137.16 103.124) (width 0.25) (layer F.Cu) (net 9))
 (segment (start 88.392 105.156) (end 90.424 103.124) (width 0.25) (layer F.Cu) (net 9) (status 10))
 (segment (start 133.54601 107.75399) (end 135.128 106.172) (width 0.25) (layer F.Cu) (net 8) (status 20))
 (segment (start 133.54601 108.26199) (end 133.54601 107.75399) (width 0.25) (layer F.Cu) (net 8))
 (segment (start 109.045999 112.315001) (end 113.09901 108.26199) (width 0.25) (layer F.Cu) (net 8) (status 10))
 (segment (start 113.09901 108.26199) (end 133.54601 108.26199) (width 0.25) (layer F.Cu) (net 8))
 (segment (start 137.668 106.172) (end 135.128 108.712) (width 0.25) (layer F.Cu) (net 7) (status 10))
 (segment (start 115.189 108.712) (end 111.585999 112.315001) (width 0.25) (layer F.Cu) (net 7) (status 20))
 (segment (start 135.128 108.712) (end 115.189 108.712) (width 0.25) (layer F.Cu) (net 7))
 (segment (start 134.366 112.395) (end 134.445999 112.315001) (width 0.25) (layer F.Cu) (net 5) (status 30))
 (segment (start 114.125999 112.315001) (end 117.221 109.22) (width 0.25) (layer B.Cu) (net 6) (status 10))
 (segment (start 129.54 109.22) (end 132.588 106.172) (width 0.25) (layer B.Cu) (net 6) (status 20))
 (segment (start 117.221 109.22) (end 129.54 109.22) (width 0.25) (layer B.Cu) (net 6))
 (segment (start 118.13 87.376) (end 119.38 87.376) (width 0.25) (layer F.Cu) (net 13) (status 20))
 (segment (start 115.824 85.07) (end 118.13 87.376) (width 0.25) (layer F.Cu) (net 13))
 (segment (start 115.824 77.216) (end 115.824 85.07) (width 0.25) (layer F.Cu) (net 13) (status 10))
 (segment (start 89.52337 97.536) (end 88.392 97.536) (width 0.25) (layer F.Cu) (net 13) (status 20))
 (segment (start 110.47 97.536) (end 89.52337 97.536) (width 0.25) (layer B.Cu) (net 13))
 (segment (start 119.38 88.626) (end 110.47 97.536) (width 0.25) (layer B.Cu) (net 13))
 (segment (start 119.38 87.376) (end 119.38 88.626) (width 0.25) (layer F.Cu) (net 13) (status 10))
 (segment (start 111.252 64.008) (end 110.744 63.5) (width 0.25) (layer F.Cu) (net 14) (status 30))
 (segment (start 111.252 69.596) (end 111.252 64.008) (width 0.25) (layer F.Cu) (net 14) (status 30))
 (segment (start 111.76 62.484) (end 110.744 63.5) (width 0.25) (layer F.Cu) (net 14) (status 20))
 (segment (start 116.332 62.484) (end 111.76 62.484) (width 0.25) (layer F.Cu) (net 14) (status 10))
 (segment (start 114.917787 57.404) (end 110.744 57.404) (width 0.25) (layer F.Cu) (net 15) (status 20))
 (segment (start 116.332 57.404) (end 114.917787 57.404) (width 0.25) (layer F.Cu) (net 15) (status 10))
 (segment (start 110.744 45.612) (end 108.68 43.548) (width 0.25) (layer F.Cu) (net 15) (status 20))
 (segment (start 110.744 57.404) (end 110.744 45.612) (width 0.25) (layer F.Cu) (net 15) (status 10))
 (segment (start 115.824 72.644) (end 111.252 77.216) (width 0.25) (layer F.Cu) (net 16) (status 20))
 (segment (start 115.824 69.596) (end 115.824 72.644) (width 0.25) (layer F.Cu) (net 16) (status 10))
 (segment (start 111.252 81.28) (end 109.728 82.804) (width 0.25) (layer F.Cu) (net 16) (status 20))
 (segment (start 111.252 77.216) (end 111.252 81.28) (width 0.25) (layer F.Cu) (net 16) (status 10))
 (segment (start 101.6 74.676) (end 106.68 69.596) (width 0.25) (layer F.Cu) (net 17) (status 20))
 (segment (start 101.6 77.216) (end 101.6 74.676) (width 0.25) (layer F.Cu) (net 17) (status 10))
 (segment (start 107.188 82.804) (end 101.6 77.216) (width 0.25) (layer F.Cu) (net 17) (status 30))
 (segment (start 140.208 97.502) (end 138.684 95.978) (width 0.25) (layer F.Cu) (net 19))
 (segment (start 140.208 98.552) (end 140.208 97.502) (width 0.25) (layer F.Cu) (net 19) (status 10))
 (segment (start 137.702 95.978) (end 137.668 96.012) (width 0.25) (layer F.Cu) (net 19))
 (segment (start 138.684 95.978) (end 137.702 95.978) (width 0.25) (layer F.Cu) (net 19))
 (segment (start 137.668 96.012) (end 135.128 98.552) (width 0.25) (layer F.Cu) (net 19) (status 20))
 (segment (start 139.158 98.552) (end 137.668 98.552) (width 0.25) (layer F.Cu) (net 19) (status 20))
 (segment (start 140.208 98.552) (end 139.158 98.552) (width 0.25) (layer F.Cu) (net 19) (status 10))
 (segment (start 127.508 88.9) (end 127.508 98.552) (width 0.25) (layer B.Cu) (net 18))
 (segment (start 122.428 83.82) (end 127.508 88.9) (width 0.25) (layer B.Cu) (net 18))
 (segment (start 106.68 77.216) (end 113.284 83.82) (width 0.25) (layer B.Cu) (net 18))
 (segment (start 113.284 83.82) (end 122.428 83.82) (width 0.25) (layer B.Cu) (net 18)))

